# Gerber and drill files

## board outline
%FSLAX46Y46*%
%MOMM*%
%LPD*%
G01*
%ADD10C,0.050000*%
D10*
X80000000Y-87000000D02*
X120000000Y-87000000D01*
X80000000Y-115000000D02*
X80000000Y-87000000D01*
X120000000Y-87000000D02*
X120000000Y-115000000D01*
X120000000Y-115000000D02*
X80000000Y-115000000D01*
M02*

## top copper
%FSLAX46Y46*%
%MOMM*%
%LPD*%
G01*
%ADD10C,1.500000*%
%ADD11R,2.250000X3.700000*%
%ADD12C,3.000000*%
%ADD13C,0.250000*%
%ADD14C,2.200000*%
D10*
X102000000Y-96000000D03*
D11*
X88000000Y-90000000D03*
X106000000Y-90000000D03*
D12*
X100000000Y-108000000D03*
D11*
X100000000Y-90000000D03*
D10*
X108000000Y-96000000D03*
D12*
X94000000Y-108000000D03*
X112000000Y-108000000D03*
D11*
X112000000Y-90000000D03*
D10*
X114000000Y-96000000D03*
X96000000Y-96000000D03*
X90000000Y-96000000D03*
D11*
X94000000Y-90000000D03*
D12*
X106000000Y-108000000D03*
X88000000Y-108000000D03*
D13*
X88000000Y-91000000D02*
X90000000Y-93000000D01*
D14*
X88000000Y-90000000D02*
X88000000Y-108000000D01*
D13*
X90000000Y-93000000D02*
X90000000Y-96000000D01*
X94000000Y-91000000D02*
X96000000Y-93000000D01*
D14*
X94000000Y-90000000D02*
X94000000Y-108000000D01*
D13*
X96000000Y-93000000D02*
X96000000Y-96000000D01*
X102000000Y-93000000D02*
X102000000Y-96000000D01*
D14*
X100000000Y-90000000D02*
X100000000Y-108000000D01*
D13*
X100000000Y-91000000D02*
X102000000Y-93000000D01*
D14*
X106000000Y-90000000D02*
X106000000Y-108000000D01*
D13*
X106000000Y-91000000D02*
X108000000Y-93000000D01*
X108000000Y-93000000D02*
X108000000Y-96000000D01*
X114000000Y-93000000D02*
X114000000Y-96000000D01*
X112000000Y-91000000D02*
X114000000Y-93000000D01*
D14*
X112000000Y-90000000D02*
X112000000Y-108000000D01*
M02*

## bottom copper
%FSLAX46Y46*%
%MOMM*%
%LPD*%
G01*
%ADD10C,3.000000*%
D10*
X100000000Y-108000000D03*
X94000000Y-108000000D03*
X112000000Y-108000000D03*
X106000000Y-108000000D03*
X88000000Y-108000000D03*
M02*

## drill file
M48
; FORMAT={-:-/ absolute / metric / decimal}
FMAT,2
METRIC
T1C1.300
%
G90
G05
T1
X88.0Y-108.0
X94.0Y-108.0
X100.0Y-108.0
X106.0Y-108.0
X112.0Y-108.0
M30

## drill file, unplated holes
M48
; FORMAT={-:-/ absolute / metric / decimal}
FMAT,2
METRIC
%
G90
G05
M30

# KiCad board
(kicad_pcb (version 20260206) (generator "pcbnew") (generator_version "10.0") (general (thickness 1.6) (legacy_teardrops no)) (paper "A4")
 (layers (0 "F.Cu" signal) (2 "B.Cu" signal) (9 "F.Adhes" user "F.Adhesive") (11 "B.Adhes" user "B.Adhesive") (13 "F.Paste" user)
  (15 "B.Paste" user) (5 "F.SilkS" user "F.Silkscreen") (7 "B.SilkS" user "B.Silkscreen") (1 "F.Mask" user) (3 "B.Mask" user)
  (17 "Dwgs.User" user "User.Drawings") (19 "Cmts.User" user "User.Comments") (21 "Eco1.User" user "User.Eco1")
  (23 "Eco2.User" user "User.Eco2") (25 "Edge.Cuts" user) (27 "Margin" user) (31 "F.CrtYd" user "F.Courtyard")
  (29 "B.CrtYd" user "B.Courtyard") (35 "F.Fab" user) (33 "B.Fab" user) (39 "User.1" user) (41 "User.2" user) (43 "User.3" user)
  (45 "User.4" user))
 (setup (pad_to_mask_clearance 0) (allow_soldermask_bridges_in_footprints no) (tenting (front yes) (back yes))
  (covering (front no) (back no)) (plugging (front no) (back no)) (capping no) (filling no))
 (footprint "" (layer "F.Cu") (at 102 96)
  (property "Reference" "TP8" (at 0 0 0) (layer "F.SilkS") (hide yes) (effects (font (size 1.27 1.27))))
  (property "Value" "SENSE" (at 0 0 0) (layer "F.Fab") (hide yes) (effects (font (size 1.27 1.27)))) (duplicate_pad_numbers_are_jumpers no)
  (pad "1" smd circle (at 0 0) (size 1.5 1.5) (layers "F.Cu" "F.Mask") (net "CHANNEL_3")))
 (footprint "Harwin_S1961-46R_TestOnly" (layer "F.Cu") (at 88 90)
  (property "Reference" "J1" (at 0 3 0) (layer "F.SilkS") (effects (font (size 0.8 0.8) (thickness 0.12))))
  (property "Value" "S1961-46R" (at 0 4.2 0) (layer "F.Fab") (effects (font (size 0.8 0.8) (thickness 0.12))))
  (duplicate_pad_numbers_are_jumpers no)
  (pad "1" smd rect (at 0 0) (size 2.25 3.7) (layers "F.Cu" "F.Mask" "F.Paste") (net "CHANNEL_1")))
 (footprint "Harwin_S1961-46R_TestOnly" (layer "F.Cu") (at 106 90)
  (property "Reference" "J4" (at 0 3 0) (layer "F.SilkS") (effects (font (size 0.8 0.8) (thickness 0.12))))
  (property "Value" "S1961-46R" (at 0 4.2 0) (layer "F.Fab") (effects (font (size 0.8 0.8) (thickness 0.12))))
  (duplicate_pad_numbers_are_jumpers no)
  (pad "1" smd rect (at 0 0) (size 2.25 3.7) (layers "F.Cu" "F.Mask" "F.Paste") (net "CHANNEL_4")))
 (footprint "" (layer "F.Cu") (at 100 108)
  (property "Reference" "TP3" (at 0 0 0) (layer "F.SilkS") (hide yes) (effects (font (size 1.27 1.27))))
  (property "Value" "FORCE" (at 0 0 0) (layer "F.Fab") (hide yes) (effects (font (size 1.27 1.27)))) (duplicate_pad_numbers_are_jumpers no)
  (pad "1" thru_hole circle (at 0 0) (size 3 3) (drill 1.3) (layers "*.Cu" "*.Mask") (remove_unused_layers no) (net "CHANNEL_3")))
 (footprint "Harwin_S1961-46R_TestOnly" (layer "F.Cu") (at 100 90)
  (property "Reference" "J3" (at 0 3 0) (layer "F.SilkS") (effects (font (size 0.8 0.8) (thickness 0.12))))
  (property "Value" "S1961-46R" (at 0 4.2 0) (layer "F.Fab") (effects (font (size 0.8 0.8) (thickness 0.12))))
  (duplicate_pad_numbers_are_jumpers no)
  (pad "1" smd rect (at 0 0) (size 2.25 3.7) (layers "F.Cu" "F.Mask" "F.Paste") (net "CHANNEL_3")))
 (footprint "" (layer "F.Cu") (at 108 96)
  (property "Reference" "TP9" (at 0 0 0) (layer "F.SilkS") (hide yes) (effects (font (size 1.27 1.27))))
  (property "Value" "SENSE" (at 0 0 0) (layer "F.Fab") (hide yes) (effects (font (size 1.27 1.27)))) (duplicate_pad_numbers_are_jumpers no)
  (pad "1" smd circle (at 0 0) (size 1.5 1.5) (layers "F.Cu" "F.Mask") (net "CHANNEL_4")))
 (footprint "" (layer "F.Cu") (at 94 108)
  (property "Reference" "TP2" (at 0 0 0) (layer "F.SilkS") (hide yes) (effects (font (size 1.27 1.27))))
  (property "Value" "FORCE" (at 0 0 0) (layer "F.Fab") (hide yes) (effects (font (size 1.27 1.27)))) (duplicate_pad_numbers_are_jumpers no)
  (pad "1" thru_hole circle (at 0 0) (size 3 3) (drill 1.3) (layers "*.Cu" "*.Mask") (remove_unused_layers no) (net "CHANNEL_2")))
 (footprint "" (layer "F.Cu") (at 112 108)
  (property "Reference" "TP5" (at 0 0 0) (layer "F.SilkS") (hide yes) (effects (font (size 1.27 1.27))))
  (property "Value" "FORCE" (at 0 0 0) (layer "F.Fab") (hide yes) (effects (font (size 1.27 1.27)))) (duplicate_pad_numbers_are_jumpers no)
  (pad "1" thru_hole circle (at 0 0) (size 3 3) (drill 1.3) (layers "*.Cu" "*.Mask") (remove_unused_layers no) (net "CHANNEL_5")))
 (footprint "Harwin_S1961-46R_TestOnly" (layer "F.Cu") (at 112 90)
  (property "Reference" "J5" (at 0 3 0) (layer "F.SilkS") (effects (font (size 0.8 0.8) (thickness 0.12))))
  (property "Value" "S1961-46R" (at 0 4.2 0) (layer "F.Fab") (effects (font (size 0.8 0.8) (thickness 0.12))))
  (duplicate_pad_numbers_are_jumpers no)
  (pad "1" smd rect (at 0 0) (size 2.25 3.7) (layers "F.Cu" "F.Mask" "F.Paste") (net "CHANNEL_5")))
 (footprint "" (layer "F.Cu") (at 114 96)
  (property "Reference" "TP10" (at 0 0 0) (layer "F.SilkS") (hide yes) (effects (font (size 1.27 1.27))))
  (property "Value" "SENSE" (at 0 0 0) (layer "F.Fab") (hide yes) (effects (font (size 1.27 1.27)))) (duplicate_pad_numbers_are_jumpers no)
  (pad "1" smd circle (at 0 0) (size 1.5 1.5) (layers "F.Cu" "F.Mask") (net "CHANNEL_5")))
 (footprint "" (layer "F.Cu") (at 96 96)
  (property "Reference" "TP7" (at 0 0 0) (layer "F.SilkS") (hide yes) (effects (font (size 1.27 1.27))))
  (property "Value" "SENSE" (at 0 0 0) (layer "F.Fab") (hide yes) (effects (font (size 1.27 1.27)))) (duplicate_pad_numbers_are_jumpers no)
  (pad "1" smd circle (at 0 0) (size 1.5 1.5) (layers "F.Cu" "F.Mask") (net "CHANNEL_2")))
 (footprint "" (layer "F.Cu") (at 90 96)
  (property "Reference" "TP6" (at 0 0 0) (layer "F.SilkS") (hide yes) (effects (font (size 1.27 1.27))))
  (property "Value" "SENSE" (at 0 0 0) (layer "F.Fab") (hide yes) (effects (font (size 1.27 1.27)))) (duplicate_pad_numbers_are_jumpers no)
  (pad "1" smd circle (at 0 0) (size 1.5 1.5) (layers "F.Cu" "F.Mask") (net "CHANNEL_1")))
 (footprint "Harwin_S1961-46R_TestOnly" (layer "F.Cu") (at 94 90)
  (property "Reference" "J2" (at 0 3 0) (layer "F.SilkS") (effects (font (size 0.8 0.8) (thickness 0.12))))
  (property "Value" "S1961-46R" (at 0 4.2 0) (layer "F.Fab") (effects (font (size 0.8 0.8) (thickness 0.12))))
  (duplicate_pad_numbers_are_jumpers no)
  (pad "1" smd rect (at 0 0) (size 2.25 3.7) (layers "F.Cu" "F.Mask" "F.Paste") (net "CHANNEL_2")))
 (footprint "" (layer "F.Cu") (at 106 108)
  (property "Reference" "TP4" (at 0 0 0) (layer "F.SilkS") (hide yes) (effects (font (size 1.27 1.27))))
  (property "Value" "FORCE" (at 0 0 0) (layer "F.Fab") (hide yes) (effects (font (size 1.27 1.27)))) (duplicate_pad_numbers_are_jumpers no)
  (pad "1" thru_hole circle (at 0 0) (size 3 3) (drill 1.3) (layers "*.Cu" "*.Mask") (remove_unused_layers no) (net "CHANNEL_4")))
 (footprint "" (layer "F.Cu") (at 88 108)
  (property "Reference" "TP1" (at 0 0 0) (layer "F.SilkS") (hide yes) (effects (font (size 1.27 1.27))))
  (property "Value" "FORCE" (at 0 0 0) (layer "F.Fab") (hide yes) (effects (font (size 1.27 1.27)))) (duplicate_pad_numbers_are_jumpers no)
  (pad "1" thru_hole circle (at 0 0) (size 3 3) (drill 1.3) (layers "*.Cu" "*.Mask") (remove_unused_layers no) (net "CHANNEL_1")))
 (gr_line (start 80 87) (end 120 87) (stroke (width 0.05) (type default)) (layer "Edge.Cuts"))
 (gr_line (start 80 115) (end 80 87) (stroke (width 0.05) (type default)) (layer "Edge.Cuts"))
 (gr_line (start 120 87) (end 120 115) (stroke (width 0.05) (type default)) (layer "Edge.Cuts"))
 (gr_line (start 120 115) (end 80 115) (stroke (width 0.05) (type default)) (layer "Edge.Cuts"))
 (segment (start 88 91) (end 90 93) (width 0.25) (layer "F.Cu") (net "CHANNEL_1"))
 (segment (start 88 90) (end 88 108) (width 2.2) (layer "F.Cu") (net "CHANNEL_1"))
 (segment (start 90 93) (end 90 96) (width 0.25) (layer "F.Cu") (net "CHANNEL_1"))
 (segment (start 94 91) (end 96 93) (width 0.25) (layer "F.Cu") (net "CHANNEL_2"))
 (segment (start 94 90) (end 94 108) (width 2.2) (layer "F.Cu") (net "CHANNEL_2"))
 (segment (start 96 93) (end 96 96) (width 0.25) (layer "F.Cu") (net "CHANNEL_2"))
 (segment (start 102 93) (end 102 96) (width 0.25) (layer "F.Cu") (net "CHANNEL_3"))
 (segment (start 100 90) (end 100 108) (width 2.2) (layer "F.Cu") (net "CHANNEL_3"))
 (segment (start 100 91) (end 102 93) (width 0.25) (layer "F.Cu") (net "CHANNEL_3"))
 (segment (start 106 90) (end 106 108) (width 2.2) (layer "F.Cu") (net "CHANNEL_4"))
 (segment (start 106 91) (end 108 93) (width 0.25) (layer "F.Cu") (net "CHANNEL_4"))
 (segment (start 108 93) (end 108 96) (width 0.25) (layer "F.Cu") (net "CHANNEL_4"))
 (segment (start 114 93) (end 114 96) (width 0.25) (layer "F.Cu") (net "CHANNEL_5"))
 (segment (start 112 91) (end 114 93) (width 0.25) (layer "F.Cu") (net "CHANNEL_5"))
 (segment (start 112 90) (end 112 108) (width 2.2) (layer "F.Cu") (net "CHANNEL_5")))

